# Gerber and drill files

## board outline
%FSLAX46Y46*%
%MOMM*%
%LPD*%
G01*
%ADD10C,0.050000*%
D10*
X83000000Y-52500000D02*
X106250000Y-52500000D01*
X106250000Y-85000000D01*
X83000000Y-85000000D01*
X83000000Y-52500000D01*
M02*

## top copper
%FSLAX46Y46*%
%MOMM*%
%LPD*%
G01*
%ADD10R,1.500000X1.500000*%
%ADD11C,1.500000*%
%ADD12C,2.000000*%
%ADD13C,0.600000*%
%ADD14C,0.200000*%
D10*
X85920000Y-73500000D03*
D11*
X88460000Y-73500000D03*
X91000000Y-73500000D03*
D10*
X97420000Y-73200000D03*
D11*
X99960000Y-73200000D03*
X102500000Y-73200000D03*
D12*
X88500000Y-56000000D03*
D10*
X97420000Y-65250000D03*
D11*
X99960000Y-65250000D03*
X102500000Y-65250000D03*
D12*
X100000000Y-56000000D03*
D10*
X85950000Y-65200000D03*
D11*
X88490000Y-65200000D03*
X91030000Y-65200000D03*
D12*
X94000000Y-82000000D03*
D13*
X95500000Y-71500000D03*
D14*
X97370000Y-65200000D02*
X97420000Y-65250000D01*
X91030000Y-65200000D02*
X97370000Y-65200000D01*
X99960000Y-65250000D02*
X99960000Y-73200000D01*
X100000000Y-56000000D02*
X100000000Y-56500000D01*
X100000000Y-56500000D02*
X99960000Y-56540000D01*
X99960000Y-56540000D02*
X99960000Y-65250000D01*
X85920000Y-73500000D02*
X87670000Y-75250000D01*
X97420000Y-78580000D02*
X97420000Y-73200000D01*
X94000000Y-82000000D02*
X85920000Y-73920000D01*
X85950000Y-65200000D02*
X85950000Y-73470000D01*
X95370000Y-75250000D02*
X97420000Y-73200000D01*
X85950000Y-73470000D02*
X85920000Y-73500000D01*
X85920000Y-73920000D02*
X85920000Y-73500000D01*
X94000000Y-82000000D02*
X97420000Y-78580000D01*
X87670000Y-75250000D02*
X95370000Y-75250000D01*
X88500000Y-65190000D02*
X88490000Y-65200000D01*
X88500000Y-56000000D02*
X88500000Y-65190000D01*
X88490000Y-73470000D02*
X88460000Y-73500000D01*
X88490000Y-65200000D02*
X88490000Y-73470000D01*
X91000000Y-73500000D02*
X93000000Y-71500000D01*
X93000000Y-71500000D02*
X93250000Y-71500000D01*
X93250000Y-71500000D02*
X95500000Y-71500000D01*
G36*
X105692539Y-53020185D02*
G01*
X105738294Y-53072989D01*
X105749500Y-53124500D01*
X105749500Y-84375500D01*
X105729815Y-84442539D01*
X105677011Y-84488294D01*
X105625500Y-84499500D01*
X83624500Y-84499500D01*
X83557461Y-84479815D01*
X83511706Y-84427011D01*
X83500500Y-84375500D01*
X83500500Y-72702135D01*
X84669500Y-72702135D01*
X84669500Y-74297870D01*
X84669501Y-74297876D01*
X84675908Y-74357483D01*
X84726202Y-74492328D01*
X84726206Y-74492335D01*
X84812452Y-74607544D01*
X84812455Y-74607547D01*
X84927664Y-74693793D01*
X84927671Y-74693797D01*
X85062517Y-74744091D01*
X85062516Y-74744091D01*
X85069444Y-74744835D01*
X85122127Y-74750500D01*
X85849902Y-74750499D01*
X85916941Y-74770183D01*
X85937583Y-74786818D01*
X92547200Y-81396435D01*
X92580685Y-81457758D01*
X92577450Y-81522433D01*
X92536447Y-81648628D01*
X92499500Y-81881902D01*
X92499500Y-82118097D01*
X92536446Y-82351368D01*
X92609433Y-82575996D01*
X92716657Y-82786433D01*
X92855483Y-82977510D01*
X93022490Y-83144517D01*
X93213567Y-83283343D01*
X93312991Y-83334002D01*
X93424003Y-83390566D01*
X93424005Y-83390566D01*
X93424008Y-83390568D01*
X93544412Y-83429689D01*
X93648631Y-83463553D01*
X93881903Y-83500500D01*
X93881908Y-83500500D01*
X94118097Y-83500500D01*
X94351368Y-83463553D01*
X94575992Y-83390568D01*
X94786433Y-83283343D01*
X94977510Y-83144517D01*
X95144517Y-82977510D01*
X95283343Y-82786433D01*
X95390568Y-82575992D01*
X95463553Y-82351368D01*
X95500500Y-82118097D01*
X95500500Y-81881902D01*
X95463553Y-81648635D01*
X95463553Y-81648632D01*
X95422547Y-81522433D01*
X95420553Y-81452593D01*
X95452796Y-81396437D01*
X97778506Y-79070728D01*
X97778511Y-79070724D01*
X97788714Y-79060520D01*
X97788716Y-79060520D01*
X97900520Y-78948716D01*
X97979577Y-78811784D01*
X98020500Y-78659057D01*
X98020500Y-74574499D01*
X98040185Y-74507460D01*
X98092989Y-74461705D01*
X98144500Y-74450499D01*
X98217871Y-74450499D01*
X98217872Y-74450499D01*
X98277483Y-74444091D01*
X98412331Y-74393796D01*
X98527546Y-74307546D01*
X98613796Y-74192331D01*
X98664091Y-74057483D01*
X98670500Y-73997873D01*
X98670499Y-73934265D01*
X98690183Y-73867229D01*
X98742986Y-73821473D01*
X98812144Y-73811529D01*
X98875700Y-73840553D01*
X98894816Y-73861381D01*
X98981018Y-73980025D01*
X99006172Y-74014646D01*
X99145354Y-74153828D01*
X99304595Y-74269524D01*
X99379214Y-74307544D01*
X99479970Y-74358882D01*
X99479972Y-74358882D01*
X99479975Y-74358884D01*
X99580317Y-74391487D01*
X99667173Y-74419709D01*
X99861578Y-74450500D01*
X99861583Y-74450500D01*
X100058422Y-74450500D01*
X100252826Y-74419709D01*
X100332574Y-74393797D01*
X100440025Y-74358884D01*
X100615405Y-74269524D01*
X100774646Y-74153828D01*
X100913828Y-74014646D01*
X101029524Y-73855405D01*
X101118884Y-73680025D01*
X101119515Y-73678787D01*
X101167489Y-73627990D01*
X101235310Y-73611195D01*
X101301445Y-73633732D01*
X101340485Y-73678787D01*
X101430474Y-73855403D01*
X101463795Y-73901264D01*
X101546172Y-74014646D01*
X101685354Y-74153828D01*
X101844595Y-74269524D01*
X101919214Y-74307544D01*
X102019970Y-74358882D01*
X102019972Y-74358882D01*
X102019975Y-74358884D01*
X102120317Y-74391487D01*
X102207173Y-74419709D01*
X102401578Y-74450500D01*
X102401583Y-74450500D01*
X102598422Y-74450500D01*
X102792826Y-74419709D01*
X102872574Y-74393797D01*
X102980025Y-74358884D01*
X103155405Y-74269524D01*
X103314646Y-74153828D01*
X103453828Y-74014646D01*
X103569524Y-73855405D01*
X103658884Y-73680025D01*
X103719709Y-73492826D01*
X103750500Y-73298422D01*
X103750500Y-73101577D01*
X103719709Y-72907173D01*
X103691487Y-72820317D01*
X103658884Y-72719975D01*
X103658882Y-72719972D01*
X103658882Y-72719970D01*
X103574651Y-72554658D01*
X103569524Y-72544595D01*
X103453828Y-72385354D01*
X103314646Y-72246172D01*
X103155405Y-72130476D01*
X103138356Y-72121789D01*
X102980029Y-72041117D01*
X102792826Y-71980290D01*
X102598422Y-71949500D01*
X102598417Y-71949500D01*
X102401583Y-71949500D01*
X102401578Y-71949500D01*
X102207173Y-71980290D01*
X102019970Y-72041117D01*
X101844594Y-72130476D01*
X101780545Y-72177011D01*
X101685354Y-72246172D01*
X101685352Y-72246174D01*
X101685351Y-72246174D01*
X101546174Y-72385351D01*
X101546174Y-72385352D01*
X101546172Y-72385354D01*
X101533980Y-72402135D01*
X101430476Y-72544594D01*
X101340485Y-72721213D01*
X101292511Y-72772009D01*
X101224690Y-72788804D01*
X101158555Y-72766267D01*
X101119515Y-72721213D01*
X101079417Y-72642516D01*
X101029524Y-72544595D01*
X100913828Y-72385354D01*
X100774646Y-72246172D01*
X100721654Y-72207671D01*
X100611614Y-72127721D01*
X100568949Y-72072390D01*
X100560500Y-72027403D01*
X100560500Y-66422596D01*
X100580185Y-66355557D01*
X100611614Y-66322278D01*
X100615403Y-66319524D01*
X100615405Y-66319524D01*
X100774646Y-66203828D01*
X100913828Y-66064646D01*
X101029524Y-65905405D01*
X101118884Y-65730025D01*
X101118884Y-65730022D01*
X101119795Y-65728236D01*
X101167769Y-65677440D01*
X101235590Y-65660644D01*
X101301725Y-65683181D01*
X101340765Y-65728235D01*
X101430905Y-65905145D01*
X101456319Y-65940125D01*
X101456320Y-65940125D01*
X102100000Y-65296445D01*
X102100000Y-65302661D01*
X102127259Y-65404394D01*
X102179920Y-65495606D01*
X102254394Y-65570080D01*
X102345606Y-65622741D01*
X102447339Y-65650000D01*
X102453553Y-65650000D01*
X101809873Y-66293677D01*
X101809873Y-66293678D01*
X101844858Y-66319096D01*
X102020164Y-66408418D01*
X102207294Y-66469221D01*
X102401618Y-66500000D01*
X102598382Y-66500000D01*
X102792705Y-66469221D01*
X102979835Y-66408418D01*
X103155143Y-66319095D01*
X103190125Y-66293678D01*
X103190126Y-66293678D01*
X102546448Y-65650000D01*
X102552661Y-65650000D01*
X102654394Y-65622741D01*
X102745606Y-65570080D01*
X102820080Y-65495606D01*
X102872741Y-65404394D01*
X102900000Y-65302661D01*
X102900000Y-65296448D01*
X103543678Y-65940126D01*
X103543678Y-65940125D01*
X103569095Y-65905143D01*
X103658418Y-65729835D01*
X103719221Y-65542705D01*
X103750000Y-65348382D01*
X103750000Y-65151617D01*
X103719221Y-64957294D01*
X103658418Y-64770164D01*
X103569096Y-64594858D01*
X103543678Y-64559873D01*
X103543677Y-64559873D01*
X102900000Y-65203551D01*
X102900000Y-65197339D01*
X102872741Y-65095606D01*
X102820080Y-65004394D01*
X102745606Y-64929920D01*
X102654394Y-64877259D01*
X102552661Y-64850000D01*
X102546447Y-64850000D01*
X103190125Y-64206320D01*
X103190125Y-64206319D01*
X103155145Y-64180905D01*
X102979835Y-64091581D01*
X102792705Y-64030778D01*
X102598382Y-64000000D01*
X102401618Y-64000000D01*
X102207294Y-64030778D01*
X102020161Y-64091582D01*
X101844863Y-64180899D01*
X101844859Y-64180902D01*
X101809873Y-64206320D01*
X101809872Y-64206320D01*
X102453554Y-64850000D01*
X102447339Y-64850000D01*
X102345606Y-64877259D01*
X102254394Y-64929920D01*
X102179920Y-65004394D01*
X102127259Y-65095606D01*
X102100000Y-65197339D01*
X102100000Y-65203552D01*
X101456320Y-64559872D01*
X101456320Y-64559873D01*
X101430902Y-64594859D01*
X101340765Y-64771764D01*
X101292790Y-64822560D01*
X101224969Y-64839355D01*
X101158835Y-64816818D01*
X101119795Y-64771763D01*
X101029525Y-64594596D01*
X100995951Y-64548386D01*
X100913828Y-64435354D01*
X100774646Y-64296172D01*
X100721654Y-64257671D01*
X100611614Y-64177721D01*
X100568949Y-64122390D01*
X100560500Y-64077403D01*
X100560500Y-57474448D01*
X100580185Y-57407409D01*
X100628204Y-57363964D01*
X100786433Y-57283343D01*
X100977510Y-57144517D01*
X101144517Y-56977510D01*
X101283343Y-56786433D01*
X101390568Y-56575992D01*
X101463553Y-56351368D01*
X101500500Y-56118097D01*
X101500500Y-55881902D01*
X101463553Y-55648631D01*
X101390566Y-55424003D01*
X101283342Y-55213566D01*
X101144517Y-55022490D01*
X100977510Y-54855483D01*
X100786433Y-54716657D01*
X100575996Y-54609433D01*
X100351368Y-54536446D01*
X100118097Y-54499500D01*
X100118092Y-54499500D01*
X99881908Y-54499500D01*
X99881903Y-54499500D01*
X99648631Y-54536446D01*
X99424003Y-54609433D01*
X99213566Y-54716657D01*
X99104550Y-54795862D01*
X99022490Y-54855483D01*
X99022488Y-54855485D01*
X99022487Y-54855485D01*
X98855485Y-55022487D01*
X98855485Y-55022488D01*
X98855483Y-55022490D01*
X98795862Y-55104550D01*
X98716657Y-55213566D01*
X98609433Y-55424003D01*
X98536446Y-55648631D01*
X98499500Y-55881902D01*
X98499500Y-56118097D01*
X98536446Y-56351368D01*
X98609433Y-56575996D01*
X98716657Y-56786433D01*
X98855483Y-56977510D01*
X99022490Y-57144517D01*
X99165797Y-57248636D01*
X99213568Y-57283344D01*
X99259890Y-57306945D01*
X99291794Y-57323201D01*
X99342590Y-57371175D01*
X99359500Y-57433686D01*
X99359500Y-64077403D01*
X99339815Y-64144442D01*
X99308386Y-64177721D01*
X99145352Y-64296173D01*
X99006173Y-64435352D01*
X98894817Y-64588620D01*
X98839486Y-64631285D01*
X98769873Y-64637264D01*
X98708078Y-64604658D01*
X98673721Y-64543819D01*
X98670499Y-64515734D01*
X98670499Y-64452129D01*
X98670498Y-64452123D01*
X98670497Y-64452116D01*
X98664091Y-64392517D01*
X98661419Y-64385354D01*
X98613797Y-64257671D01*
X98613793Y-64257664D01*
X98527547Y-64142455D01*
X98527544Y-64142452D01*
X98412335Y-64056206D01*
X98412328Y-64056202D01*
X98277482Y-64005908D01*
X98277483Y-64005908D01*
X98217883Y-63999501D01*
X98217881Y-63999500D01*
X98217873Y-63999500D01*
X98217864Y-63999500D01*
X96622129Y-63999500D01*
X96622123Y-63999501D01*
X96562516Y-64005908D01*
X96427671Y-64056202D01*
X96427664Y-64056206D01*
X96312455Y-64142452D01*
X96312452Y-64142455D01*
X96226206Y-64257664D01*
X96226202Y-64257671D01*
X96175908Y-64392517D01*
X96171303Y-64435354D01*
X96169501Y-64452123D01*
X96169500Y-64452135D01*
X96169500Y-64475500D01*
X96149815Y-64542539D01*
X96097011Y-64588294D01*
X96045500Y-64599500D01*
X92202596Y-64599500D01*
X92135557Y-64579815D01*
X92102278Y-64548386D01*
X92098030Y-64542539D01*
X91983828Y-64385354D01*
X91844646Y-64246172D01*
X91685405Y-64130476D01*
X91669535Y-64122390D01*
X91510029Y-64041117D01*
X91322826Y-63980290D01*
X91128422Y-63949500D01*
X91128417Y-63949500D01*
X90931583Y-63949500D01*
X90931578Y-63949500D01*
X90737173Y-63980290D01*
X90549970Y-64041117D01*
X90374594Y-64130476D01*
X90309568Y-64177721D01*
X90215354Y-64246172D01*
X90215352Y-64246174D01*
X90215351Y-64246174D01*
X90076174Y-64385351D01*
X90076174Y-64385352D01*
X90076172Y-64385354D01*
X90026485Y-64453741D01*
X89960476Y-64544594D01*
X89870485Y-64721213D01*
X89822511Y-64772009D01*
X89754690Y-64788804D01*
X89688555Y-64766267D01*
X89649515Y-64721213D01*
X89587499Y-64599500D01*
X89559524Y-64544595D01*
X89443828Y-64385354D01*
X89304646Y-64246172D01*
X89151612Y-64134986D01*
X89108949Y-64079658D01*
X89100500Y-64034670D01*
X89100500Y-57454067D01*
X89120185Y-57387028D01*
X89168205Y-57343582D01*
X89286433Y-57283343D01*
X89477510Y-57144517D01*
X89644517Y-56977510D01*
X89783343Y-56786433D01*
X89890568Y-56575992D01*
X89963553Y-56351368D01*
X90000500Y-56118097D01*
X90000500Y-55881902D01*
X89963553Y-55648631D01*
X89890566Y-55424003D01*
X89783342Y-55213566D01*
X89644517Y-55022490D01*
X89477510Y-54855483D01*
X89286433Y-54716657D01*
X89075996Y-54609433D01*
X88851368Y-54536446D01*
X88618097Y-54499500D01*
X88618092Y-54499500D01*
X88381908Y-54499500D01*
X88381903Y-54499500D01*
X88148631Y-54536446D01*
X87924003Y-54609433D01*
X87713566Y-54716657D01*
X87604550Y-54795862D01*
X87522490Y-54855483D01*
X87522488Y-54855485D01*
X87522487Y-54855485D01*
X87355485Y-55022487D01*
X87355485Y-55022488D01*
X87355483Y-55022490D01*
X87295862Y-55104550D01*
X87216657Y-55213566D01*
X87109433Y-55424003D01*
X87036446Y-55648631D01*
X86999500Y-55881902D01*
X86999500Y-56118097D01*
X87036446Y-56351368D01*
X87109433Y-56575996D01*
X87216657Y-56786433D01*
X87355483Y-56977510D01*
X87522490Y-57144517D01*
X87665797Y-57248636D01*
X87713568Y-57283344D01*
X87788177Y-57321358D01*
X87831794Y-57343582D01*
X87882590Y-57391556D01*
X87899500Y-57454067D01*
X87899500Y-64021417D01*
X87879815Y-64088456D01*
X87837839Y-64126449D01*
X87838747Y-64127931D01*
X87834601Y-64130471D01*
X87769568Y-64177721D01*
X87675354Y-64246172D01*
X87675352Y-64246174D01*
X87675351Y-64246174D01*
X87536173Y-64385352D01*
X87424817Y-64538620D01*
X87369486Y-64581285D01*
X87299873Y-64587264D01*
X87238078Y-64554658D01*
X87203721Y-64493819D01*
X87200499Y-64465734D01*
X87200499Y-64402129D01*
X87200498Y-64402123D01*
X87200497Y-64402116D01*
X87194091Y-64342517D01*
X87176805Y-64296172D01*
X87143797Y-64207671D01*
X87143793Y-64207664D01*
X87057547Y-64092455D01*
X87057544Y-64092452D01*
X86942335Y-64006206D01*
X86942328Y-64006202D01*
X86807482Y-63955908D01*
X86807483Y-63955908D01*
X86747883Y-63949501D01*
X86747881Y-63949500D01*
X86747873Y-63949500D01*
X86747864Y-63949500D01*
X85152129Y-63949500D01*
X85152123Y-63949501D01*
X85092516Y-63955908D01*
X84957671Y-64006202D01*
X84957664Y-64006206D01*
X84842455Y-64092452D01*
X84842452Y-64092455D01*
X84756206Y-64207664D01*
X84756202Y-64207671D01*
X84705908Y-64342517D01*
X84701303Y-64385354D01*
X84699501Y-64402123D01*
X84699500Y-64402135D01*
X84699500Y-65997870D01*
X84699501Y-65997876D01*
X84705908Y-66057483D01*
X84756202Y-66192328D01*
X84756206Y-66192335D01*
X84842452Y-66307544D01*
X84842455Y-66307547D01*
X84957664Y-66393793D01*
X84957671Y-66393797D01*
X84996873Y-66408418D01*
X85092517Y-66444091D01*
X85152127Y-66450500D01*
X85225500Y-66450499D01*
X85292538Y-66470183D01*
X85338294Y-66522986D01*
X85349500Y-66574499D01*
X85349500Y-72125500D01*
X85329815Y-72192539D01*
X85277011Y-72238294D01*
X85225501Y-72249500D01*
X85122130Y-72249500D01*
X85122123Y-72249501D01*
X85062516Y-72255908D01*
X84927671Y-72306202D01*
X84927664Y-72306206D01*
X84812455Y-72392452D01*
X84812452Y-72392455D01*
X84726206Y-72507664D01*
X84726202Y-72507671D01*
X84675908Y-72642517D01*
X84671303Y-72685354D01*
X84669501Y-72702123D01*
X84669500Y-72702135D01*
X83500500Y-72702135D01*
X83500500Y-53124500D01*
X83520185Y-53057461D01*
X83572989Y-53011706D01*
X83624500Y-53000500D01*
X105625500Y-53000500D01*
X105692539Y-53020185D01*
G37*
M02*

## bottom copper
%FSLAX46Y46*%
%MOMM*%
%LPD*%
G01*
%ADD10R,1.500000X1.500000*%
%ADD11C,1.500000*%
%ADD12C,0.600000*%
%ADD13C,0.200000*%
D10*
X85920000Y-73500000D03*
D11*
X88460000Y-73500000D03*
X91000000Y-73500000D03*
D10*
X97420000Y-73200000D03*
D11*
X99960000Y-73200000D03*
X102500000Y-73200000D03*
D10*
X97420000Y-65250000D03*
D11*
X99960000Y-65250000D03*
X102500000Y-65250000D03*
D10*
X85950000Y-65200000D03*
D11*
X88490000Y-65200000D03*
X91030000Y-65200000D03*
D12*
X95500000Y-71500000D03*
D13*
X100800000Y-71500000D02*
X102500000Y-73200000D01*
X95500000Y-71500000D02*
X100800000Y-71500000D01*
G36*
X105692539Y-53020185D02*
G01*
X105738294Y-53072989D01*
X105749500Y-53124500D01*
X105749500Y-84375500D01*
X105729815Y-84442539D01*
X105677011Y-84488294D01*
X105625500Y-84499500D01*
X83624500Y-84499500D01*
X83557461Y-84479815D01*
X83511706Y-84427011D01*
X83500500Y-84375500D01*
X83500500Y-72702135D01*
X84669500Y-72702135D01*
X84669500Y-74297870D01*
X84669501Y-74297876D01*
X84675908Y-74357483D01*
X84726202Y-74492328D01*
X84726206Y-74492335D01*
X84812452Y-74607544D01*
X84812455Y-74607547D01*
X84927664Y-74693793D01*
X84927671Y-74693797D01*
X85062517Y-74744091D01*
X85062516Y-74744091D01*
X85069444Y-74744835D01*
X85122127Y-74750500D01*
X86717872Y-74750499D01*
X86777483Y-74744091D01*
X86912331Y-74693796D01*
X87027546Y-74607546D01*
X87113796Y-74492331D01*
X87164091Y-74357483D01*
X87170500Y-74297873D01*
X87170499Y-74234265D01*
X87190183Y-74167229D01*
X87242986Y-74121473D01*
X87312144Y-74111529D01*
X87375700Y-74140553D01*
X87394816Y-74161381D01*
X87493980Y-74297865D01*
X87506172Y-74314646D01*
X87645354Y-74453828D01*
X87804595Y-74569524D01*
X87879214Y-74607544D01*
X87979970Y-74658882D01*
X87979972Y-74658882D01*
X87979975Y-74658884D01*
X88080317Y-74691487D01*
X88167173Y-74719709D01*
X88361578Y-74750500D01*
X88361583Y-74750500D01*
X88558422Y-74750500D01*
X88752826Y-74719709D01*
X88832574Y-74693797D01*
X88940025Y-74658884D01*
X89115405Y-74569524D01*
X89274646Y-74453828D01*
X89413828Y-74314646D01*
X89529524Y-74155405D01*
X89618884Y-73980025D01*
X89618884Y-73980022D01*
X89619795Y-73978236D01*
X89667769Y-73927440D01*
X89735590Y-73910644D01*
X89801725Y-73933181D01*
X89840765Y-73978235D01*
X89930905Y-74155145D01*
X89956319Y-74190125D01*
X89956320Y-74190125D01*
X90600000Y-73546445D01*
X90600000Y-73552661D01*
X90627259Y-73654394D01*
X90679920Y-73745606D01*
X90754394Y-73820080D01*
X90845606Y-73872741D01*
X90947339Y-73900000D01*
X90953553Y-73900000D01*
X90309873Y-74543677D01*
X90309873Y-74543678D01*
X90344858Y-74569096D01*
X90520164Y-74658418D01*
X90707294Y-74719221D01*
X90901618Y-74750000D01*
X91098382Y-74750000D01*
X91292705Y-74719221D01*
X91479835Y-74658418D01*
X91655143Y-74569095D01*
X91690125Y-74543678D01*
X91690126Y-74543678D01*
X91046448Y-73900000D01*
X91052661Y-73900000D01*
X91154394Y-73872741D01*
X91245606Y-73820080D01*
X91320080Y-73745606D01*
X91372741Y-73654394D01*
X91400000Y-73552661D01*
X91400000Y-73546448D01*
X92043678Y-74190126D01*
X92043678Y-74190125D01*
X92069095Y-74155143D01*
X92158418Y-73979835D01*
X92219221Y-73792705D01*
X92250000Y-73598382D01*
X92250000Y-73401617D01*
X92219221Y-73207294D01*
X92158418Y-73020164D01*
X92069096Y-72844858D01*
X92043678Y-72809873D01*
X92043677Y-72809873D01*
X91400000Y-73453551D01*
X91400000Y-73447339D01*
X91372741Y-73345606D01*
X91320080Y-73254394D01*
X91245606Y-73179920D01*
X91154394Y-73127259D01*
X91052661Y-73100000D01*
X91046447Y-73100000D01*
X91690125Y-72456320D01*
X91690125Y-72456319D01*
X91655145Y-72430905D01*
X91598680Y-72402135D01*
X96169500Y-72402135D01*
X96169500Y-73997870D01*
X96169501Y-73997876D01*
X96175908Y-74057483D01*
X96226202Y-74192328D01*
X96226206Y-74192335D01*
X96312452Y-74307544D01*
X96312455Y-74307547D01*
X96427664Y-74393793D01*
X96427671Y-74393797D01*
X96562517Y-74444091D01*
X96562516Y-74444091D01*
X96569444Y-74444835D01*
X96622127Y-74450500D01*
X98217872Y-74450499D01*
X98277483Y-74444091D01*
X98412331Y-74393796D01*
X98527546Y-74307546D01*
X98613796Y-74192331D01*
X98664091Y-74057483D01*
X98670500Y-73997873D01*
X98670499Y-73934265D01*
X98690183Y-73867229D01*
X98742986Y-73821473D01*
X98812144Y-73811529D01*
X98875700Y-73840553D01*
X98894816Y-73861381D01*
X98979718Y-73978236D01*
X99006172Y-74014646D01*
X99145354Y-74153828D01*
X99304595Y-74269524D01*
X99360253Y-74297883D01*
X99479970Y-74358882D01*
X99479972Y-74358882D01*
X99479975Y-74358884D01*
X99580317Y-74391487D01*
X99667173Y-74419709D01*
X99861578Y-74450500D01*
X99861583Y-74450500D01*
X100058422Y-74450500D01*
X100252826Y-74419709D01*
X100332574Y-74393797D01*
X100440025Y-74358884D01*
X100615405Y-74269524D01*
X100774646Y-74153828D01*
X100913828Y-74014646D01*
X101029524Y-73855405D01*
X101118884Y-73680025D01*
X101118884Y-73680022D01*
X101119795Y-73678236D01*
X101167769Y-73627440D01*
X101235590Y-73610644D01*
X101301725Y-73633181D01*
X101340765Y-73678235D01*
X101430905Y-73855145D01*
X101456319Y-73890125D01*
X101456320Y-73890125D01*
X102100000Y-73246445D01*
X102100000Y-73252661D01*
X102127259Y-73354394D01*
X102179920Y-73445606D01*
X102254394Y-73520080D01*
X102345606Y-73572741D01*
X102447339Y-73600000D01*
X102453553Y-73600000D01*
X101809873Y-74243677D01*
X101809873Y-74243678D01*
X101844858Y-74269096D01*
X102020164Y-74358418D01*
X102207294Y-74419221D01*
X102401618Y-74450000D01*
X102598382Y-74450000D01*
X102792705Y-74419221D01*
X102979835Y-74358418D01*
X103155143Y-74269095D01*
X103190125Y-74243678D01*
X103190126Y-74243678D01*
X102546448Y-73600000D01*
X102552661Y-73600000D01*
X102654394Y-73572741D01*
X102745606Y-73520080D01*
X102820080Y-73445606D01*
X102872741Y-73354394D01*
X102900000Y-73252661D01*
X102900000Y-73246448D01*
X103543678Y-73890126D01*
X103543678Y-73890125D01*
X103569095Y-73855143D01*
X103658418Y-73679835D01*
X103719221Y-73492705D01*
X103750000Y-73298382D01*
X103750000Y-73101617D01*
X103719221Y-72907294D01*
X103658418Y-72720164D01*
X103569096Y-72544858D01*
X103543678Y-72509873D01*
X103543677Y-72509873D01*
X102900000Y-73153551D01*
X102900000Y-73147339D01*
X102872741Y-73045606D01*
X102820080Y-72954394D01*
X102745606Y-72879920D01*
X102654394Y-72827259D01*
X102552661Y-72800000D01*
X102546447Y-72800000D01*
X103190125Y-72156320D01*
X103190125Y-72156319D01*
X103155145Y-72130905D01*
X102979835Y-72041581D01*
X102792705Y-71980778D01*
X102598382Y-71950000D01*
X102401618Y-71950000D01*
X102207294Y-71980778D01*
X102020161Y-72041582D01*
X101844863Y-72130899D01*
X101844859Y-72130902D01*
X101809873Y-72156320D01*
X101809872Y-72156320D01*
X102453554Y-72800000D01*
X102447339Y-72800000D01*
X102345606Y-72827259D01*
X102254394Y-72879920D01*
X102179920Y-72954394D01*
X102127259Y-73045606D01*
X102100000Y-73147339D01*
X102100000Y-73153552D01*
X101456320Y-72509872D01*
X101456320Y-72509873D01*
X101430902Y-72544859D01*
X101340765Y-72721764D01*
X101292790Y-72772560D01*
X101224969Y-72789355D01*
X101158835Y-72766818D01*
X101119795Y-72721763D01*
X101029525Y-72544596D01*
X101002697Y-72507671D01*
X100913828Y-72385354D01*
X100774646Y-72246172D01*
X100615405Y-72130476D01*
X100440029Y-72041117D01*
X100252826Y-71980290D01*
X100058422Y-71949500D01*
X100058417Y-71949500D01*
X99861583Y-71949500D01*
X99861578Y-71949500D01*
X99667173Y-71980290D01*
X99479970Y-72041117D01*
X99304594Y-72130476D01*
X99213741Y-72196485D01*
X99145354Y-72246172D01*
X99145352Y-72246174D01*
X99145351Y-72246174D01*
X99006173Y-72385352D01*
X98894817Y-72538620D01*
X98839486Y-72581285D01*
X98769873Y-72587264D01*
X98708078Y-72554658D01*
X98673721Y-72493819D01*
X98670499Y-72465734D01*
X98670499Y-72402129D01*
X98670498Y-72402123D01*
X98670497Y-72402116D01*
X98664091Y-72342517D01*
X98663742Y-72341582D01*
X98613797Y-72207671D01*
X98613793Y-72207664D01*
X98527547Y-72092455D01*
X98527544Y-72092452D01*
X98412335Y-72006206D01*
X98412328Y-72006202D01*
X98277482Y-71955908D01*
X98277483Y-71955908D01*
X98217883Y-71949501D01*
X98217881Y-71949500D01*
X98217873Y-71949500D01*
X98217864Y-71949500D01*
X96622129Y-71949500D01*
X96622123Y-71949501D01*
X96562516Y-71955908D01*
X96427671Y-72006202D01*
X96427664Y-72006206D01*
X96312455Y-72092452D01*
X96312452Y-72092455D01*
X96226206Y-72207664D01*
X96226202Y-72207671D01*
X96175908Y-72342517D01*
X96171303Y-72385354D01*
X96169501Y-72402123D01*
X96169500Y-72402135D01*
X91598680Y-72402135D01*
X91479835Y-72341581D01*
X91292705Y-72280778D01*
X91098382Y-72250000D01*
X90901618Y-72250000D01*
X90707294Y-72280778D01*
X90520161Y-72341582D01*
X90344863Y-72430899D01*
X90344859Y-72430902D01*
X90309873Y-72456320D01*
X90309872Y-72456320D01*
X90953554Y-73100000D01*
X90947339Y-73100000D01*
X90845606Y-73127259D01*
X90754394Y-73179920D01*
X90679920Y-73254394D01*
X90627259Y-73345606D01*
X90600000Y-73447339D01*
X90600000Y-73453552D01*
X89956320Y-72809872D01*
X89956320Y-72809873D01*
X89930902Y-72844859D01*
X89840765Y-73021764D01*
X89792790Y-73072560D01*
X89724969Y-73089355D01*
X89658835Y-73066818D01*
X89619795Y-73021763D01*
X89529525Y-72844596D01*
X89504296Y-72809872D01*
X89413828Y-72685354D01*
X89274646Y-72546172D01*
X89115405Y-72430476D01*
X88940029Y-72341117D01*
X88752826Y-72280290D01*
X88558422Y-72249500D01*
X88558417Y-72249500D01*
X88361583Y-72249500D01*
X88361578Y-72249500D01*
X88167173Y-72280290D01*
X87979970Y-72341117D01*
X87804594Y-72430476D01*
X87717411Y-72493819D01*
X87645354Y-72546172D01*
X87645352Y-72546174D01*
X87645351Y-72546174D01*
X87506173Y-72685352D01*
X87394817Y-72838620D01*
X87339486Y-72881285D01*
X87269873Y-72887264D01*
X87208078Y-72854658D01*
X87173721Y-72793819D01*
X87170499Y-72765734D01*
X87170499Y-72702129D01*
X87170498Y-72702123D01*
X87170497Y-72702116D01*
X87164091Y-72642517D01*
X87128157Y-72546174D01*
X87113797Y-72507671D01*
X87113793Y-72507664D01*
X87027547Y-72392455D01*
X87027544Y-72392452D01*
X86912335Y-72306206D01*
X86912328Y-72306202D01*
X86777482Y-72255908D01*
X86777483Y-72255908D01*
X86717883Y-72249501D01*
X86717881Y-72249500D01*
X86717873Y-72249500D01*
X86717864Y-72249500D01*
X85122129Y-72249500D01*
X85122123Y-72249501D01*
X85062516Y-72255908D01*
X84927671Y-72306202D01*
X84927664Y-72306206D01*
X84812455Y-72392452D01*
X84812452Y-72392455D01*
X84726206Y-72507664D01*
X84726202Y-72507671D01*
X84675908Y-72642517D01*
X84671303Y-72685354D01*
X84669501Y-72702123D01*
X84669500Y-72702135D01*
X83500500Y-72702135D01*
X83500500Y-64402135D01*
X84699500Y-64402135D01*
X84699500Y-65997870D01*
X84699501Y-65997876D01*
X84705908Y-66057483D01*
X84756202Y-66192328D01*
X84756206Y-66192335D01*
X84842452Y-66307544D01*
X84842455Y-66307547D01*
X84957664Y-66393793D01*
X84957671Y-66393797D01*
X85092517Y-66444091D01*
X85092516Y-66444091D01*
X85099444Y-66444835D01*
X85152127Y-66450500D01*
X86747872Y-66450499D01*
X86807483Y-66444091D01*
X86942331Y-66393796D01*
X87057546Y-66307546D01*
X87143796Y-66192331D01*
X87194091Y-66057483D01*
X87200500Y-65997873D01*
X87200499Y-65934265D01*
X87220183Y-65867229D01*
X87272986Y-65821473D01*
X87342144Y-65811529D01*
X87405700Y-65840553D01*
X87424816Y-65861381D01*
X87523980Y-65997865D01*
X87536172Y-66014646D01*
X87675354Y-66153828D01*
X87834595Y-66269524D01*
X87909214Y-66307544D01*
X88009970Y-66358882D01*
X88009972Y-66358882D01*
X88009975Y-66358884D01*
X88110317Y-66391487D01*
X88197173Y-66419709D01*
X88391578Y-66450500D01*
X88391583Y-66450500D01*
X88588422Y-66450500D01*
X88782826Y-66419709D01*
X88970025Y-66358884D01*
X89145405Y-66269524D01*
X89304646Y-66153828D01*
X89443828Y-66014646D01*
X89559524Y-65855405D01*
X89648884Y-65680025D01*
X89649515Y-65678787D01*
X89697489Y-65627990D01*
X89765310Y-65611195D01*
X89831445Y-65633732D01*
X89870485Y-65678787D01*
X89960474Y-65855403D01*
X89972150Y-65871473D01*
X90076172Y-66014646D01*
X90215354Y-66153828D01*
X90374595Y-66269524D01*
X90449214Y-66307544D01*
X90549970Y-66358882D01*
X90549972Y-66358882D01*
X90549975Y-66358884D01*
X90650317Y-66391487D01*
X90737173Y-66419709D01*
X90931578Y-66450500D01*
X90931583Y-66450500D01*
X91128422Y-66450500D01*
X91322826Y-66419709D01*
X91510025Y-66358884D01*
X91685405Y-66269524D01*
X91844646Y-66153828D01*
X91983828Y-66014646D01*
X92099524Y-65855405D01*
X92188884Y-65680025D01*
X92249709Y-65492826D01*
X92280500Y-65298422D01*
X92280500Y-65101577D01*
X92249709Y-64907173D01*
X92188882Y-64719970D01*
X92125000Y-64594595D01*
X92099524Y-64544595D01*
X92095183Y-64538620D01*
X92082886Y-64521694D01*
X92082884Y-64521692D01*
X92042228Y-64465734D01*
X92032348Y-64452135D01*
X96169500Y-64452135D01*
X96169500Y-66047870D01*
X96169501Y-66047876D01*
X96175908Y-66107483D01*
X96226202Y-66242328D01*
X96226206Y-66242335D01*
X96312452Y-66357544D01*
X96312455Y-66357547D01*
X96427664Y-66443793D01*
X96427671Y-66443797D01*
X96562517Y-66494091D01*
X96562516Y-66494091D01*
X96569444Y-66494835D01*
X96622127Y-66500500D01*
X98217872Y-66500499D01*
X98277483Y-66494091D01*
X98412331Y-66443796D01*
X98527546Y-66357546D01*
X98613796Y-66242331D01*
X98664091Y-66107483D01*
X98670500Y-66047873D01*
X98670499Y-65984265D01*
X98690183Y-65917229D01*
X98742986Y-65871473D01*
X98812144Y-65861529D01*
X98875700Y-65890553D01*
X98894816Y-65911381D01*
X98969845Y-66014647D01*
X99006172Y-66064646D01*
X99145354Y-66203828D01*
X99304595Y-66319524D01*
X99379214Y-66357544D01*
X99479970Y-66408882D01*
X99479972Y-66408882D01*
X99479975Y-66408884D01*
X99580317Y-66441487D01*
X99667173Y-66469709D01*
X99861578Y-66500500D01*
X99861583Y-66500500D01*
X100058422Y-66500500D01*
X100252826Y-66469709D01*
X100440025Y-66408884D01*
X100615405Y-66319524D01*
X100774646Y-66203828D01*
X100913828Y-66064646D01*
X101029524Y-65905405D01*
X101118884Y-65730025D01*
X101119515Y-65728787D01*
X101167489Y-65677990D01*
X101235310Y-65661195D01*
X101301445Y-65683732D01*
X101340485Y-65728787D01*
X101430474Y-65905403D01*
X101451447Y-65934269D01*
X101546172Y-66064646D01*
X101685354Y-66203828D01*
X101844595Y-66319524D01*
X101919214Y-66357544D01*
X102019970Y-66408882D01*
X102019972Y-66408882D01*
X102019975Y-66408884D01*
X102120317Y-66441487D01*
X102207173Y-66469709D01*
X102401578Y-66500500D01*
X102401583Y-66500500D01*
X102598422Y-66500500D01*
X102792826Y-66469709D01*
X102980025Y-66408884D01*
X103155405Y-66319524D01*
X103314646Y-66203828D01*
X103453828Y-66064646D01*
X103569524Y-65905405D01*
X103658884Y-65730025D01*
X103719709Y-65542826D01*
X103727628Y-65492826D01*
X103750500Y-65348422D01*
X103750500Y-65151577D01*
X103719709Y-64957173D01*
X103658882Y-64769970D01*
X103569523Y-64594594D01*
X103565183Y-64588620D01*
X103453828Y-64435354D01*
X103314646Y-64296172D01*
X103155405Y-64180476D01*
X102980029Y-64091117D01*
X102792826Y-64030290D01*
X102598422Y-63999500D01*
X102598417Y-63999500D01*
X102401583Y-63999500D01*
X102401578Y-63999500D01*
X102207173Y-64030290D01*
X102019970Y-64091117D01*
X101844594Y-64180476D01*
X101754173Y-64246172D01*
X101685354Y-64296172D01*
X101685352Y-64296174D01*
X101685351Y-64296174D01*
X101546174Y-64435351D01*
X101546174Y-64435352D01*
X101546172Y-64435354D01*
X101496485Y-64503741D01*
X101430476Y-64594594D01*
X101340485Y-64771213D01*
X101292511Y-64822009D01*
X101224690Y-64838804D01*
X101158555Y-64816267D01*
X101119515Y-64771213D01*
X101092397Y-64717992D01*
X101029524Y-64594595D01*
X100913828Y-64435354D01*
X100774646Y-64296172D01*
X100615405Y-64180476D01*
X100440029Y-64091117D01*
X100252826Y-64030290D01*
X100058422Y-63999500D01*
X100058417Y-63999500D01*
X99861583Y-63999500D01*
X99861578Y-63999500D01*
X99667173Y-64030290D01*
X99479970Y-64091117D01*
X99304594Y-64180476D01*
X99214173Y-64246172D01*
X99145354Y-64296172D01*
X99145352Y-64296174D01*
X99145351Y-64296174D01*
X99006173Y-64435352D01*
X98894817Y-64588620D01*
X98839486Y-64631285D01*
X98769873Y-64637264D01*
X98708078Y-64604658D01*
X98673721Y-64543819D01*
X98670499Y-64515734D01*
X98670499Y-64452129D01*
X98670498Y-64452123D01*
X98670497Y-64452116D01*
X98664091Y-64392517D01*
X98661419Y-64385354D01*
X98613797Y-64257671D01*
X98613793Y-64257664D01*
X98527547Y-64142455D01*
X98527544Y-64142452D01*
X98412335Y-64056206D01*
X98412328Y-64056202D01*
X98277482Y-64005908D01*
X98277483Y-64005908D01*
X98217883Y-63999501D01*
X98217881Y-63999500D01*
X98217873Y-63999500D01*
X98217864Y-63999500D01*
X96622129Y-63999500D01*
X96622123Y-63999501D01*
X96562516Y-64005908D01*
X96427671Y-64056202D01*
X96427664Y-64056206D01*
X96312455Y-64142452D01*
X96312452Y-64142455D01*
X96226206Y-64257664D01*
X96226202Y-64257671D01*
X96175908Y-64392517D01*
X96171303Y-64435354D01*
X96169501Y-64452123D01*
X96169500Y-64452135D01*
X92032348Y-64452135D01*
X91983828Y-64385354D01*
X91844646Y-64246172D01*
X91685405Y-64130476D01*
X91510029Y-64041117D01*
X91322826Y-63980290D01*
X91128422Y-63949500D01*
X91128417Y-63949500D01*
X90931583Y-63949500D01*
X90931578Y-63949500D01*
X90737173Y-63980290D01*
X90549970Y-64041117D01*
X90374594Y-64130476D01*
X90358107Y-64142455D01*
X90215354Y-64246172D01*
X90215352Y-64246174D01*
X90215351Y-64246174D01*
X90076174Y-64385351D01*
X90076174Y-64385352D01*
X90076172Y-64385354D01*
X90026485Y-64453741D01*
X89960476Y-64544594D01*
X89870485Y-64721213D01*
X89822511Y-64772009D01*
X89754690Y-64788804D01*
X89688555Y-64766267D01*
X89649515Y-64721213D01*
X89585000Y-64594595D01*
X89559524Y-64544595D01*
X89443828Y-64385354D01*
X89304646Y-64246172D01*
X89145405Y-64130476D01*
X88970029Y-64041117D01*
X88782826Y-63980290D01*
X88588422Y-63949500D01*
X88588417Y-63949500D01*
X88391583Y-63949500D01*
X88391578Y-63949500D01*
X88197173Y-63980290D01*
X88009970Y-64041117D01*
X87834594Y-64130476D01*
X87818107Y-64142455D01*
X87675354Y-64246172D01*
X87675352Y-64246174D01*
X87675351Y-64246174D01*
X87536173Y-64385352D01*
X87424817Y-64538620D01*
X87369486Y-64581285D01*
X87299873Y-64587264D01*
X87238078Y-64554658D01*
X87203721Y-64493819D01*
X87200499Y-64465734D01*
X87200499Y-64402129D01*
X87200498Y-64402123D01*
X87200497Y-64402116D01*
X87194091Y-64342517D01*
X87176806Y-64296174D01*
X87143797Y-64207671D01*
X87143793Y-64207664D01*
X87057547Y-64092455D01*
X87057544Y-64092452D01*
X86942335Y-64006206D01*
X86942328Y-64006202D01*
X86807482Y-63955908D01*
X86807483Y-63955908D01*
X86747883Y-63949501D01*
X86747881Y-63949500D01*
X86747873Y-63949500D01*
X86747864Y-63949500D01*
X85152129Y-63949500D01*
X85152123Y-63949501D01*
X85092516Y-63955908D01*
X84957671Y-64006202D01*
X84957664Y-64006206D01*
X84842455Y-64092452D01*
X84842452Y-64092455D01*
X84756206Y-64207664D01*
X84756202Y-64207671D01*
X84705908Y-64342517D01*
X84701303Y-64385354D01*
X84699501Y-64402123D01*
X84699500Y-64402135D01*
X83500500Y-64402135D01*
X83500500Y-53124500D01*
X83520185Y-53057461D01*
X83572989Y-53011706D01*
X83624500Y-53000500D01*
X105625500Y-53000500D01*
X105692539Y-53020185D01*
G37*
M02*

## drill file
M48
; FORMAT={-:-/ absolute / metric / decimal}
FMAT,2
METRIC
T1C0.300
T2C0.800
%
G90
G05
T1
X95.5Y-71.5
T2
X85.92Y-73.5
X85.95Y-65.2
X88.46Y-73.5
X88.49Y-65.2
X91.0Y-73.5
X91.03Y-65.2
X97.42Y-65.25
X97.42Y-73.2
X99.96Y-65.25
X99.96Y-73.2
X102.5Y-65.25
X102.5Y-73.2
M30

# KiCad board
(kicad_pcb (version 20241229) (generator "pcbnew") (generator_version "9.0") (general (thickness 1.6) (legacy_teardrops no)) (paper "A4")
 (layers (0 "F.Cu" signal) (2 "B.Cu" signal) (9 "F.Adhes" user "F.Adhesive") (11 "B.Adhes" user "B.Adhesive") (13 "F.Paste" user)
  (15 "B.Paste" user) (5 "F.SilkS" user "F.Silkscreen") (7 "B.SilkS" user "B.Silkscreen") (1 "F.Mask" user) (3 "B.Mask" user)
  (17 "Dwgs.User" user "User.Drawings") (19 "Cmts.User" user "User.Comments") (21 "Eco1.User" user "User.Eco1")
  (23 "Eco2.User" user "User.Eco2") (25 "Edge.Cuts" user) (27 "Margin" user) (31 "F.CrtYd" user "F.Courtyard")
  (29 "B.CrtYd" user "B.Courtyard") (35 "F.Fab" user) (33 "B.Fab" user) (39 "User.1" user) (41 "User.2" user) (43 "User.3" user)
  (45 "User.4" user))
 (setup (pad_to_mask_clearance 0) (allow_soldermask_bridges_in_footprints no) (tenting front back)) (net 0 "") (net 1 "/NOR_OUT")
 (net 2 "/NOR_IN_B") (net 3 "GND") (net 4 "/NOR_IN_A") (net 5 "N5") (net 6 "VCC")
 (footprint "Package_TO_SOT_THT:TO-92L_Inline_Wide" (layer "F.Cu") (at 85.92 73.5)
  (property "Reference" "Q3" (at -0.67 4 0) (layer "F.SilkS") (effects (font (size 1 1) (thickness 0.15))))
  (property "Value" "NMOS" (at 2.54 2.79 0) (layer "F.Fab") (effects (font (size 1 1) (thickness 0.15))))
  (pad "1" thru_hole rect (at 0 0) (size 1.5 1.5) (drill 0.8) (layers "*.Cu" "*.Mask") (remove_unused_layers no) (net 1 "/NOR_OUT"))
  (pad "2" thru_hole circle (at 2.54 0) (size 1.5 1.5) (drill 0.8) (layers "*.Cu" "*.Mask") (remove_unused_layers no) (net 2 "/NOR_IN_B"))
  (pad "3" thru_hole circle (at 5.08 0) (size 1.5 1.5) (drill 0.8) (layers "*.Cu" "*.Mask") (remove_unused_layers no) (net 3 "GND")))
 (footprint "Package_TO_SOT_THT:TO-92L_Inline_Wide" (layer "F.Cu") (at 97.42 73.2)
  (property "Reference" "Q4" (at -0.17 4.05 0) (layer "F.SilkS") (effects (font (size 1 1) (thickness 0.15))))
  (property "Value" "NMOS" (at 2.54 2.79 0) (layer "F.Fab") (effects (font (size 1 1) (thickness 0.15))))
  (pad "1" thru_hole rect (at 0 0) (size 1.5 1.5) (drill 0.8) (layers "*.Cu" "*.Mask") (remove_unused_layers no) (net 1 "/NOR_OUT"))
  (pad "2" thru_hole circle (at 2.54 0) (size 1.5 1.5) (drill 0.8) (layers "*.Cu" "*.Mask") (remove_unused_layers no) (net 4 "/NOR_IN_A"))
  (pad "3" thru_hole circle (at 5.08 0) (size 1.5 1.5) (drill 0.8) (layers "*.Cu" "*.Mask") (remove_unused_layers no) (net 3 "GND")))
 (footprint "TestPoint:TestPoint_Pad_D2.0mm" (layer "F.Cu") (at 88.5 56)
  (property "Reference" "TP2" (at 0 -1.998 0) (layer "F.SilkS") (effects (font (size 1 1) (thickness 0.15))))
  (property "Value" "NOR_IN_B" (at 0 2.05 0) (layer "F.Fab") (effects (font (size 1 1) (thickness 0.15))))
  (pad "1" smd circle (at 0 0) (size 2 2) (layers "F.Cu" "F.Mask") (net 2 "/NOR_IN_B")))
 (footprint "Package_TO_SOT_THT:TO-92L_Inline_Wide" (layer "F.Cu") (at 97.42 65.25)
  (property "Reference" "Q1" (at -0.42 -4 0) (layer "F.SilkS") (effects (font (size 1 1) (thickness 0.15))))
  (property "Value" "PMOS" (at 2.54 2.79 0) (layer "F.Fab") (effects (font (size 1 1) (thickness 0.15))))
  (pad "1" thru_hole rect (at 0 0) (size 1.5 1.5) (drill 0.8) (layers "*.Cu" "*.Mask") (remove_unused_layers no) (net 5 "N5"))
  (pad "2" thru_hole circle (at 2.54 0) (size 1.5 1.5) (drill 0.8) (layers "*.Cu" "*.Mask") (remove_unused_layers no) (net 4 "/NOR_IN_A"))
  (pad "3" thru_hole circle (at 5.08 0) (size 1.5 1.5) (drill 0.8) (layers "*.Cu" "*.Mask") (remove_unused_layers no) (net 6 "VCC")))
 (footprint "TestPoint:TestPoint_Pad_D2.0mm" (layer "F.Cu") (at 100 56)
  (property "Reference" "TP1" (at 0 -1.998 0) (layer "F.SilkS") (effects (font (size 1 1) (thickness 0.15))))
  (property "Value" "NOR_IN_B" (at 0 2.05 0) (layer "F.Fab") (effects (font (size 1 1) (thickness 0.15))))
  (pad "1" smd circle (at 0 0) (size 2 2) (layers "F.Cu" "F.Mask") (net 4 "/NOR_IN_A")))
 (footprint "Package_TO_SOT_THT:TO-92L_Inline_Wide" (layer "F.Cu") (at 85.95 65.2)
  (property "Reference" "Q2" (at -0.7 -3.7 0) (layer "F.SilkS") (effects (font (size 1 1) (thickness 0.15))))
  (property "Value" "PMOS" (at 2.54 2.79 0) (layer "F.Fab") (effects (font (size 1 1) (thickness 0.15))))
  (pad "1" thru_hole rect (at 0 0) (size 1.5 1.5) (drill 0.8) (layers "*.Cu" "*.Mask") (remove_unused_layers no) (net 1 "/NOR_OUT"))
  (pad "2" thru_hole circle (at 2.54 0) (size 1.5 1.5) (drill 0.8) (layers "*.Cu" "*.Mask") (remove_unused_layers no) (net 2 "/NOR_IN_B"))
  (pad "3" thru_hole circle (at 5.08 0) (size 1.5 1.5) (drill 0.8) (layers "*.Cu" "*.Mask") (remove_unused_layers no) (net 5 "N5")))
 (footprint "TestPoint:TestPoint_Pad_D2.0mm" (layer "F.Cu") (at 94 82)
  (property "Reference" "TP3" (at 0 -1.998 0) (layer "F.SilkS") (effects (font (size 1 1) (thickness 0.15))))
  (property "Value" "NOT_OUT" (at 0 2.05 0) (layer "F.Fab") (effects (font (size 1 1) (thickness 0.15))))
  (pad "1" smd circle (at 0 0) (size 2 2) (layers "F.Cu" "F.Mask") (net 1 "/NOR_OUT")))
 (gr_rect (start 83 52.5) (end 106.25 85) (stroke (width 0.05) (type default)) (fill no) (layer "Edge.Cuts"))
 (segment (start 97.37 65.2) (end 97.42 65.25) (width 0.2) (layer "F.Cu") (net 5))
 (segment (start 91.03 65.2) (end 97.37 65.2) (width 0.2) (layer "F.Cu") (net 5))
 (segment (start 99.96 65.25) (end 99.96 73.2) (width 0.2) (layer "F.Cu") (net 4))
 (segment (start 100 56) (end 100 56.5) (width 0.2) (layer "F.Cu") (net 4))
 (segment (start 100 56.5) (end 99.96 56.54) (width 0.2) (layer "F.Cu") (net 4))
 (segment (start 99.96 56.54) (end 99.96 65.25) (width 0.2) (layer "F.Cu") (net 4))
 (segment (start 85.92 73.5) (end 87.67 75.25) (width 0.2) (layer "F.Cu") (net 1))
 (segment (start 97.42 78.58) (end 97.42 73.2) (width 0.2) (layer "F.Cu") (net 1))
 (segment (start 94 82) (end 85.92 73.92) (width 0.2) (layer "F.Cu") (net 1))
 (segment (start 85.95 65.2) (end 85.95 73.47) (width 0.2) (layer "F.Cu") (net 1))
 (segment (start 95.37 75.25) (end 97.42 73.2) (width 0.2) (layer "F.Cu") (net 1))
 (segment (start 85.95 73.47) (end 85.92 73.5) (width 0.2) (layer "F.Cu") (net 1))
 (segment (start 85.92 73.92) (end 85.92 73.5) (width 0.2) (layer "F.Cu") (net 1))
 (segment (start 94 82) (end 97.42 78.58) (width 0.2) (layer "F.Cu") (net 1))
 (segment (start 87.67 75.25) (end 95.37 75.25) (width 0.2) (layer "F.Cu") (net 1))
 (segment (start 88.5 65.19) (end 88.49 65.2) (width 0.2) (layer "F.Cu") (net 2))
 (segment (start 88.5 56) (end 88.5 65.19) (width 0.2) (layer "F.Cu") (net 2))
 (segment (start 88.49 73.47) (end 88.46 73.5) (width 0.2) (layer "F.Cu") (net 2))
 (segment (start 88.49 65.2) (end 88.49 73.47) (width 0.2) (layer "F.Cu") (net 2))
 (segment (start 91 73.5) (end 93 71.5) (width 0.2) (layer "F.Cu") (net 3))
 (segment (start 93 71.5) (end 93.25 71.5) (width 0.2) (layer "F.Cu") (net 3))
 (segment (start 93.25 71.5) (end 95.5 71.5) (width 0.2) (layer "F.Cu") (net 3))
 (via (at 95.5 71.5) (size 0.6) (drill 0.3) (layers "F.Cu" "B.Cu") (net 3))
 (segment (start 100.8 71.5) (end 102.5 73.2) (width 0.2) (layer "B.Cu") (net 3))
 (segment (start 95.5 71.5) (end 100.8 71.5) (width 0.2) (layer "B.Cu") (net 3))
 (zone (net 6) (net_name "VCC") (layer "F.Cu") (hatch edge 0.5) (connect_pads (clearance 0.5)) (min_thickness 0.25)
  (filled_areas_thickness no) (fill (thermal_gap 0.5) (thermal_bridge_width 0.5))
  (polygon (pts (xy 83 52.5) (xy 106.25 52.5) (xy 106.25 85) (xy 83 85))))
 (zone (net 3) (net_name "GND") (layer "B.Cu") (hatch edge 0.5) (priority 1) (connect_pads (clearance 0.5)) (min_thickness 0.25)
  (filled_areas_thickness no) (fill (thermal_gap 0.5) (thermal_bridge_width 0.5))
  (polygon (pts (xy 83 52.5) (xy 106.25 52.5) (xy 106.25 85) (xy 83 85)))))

